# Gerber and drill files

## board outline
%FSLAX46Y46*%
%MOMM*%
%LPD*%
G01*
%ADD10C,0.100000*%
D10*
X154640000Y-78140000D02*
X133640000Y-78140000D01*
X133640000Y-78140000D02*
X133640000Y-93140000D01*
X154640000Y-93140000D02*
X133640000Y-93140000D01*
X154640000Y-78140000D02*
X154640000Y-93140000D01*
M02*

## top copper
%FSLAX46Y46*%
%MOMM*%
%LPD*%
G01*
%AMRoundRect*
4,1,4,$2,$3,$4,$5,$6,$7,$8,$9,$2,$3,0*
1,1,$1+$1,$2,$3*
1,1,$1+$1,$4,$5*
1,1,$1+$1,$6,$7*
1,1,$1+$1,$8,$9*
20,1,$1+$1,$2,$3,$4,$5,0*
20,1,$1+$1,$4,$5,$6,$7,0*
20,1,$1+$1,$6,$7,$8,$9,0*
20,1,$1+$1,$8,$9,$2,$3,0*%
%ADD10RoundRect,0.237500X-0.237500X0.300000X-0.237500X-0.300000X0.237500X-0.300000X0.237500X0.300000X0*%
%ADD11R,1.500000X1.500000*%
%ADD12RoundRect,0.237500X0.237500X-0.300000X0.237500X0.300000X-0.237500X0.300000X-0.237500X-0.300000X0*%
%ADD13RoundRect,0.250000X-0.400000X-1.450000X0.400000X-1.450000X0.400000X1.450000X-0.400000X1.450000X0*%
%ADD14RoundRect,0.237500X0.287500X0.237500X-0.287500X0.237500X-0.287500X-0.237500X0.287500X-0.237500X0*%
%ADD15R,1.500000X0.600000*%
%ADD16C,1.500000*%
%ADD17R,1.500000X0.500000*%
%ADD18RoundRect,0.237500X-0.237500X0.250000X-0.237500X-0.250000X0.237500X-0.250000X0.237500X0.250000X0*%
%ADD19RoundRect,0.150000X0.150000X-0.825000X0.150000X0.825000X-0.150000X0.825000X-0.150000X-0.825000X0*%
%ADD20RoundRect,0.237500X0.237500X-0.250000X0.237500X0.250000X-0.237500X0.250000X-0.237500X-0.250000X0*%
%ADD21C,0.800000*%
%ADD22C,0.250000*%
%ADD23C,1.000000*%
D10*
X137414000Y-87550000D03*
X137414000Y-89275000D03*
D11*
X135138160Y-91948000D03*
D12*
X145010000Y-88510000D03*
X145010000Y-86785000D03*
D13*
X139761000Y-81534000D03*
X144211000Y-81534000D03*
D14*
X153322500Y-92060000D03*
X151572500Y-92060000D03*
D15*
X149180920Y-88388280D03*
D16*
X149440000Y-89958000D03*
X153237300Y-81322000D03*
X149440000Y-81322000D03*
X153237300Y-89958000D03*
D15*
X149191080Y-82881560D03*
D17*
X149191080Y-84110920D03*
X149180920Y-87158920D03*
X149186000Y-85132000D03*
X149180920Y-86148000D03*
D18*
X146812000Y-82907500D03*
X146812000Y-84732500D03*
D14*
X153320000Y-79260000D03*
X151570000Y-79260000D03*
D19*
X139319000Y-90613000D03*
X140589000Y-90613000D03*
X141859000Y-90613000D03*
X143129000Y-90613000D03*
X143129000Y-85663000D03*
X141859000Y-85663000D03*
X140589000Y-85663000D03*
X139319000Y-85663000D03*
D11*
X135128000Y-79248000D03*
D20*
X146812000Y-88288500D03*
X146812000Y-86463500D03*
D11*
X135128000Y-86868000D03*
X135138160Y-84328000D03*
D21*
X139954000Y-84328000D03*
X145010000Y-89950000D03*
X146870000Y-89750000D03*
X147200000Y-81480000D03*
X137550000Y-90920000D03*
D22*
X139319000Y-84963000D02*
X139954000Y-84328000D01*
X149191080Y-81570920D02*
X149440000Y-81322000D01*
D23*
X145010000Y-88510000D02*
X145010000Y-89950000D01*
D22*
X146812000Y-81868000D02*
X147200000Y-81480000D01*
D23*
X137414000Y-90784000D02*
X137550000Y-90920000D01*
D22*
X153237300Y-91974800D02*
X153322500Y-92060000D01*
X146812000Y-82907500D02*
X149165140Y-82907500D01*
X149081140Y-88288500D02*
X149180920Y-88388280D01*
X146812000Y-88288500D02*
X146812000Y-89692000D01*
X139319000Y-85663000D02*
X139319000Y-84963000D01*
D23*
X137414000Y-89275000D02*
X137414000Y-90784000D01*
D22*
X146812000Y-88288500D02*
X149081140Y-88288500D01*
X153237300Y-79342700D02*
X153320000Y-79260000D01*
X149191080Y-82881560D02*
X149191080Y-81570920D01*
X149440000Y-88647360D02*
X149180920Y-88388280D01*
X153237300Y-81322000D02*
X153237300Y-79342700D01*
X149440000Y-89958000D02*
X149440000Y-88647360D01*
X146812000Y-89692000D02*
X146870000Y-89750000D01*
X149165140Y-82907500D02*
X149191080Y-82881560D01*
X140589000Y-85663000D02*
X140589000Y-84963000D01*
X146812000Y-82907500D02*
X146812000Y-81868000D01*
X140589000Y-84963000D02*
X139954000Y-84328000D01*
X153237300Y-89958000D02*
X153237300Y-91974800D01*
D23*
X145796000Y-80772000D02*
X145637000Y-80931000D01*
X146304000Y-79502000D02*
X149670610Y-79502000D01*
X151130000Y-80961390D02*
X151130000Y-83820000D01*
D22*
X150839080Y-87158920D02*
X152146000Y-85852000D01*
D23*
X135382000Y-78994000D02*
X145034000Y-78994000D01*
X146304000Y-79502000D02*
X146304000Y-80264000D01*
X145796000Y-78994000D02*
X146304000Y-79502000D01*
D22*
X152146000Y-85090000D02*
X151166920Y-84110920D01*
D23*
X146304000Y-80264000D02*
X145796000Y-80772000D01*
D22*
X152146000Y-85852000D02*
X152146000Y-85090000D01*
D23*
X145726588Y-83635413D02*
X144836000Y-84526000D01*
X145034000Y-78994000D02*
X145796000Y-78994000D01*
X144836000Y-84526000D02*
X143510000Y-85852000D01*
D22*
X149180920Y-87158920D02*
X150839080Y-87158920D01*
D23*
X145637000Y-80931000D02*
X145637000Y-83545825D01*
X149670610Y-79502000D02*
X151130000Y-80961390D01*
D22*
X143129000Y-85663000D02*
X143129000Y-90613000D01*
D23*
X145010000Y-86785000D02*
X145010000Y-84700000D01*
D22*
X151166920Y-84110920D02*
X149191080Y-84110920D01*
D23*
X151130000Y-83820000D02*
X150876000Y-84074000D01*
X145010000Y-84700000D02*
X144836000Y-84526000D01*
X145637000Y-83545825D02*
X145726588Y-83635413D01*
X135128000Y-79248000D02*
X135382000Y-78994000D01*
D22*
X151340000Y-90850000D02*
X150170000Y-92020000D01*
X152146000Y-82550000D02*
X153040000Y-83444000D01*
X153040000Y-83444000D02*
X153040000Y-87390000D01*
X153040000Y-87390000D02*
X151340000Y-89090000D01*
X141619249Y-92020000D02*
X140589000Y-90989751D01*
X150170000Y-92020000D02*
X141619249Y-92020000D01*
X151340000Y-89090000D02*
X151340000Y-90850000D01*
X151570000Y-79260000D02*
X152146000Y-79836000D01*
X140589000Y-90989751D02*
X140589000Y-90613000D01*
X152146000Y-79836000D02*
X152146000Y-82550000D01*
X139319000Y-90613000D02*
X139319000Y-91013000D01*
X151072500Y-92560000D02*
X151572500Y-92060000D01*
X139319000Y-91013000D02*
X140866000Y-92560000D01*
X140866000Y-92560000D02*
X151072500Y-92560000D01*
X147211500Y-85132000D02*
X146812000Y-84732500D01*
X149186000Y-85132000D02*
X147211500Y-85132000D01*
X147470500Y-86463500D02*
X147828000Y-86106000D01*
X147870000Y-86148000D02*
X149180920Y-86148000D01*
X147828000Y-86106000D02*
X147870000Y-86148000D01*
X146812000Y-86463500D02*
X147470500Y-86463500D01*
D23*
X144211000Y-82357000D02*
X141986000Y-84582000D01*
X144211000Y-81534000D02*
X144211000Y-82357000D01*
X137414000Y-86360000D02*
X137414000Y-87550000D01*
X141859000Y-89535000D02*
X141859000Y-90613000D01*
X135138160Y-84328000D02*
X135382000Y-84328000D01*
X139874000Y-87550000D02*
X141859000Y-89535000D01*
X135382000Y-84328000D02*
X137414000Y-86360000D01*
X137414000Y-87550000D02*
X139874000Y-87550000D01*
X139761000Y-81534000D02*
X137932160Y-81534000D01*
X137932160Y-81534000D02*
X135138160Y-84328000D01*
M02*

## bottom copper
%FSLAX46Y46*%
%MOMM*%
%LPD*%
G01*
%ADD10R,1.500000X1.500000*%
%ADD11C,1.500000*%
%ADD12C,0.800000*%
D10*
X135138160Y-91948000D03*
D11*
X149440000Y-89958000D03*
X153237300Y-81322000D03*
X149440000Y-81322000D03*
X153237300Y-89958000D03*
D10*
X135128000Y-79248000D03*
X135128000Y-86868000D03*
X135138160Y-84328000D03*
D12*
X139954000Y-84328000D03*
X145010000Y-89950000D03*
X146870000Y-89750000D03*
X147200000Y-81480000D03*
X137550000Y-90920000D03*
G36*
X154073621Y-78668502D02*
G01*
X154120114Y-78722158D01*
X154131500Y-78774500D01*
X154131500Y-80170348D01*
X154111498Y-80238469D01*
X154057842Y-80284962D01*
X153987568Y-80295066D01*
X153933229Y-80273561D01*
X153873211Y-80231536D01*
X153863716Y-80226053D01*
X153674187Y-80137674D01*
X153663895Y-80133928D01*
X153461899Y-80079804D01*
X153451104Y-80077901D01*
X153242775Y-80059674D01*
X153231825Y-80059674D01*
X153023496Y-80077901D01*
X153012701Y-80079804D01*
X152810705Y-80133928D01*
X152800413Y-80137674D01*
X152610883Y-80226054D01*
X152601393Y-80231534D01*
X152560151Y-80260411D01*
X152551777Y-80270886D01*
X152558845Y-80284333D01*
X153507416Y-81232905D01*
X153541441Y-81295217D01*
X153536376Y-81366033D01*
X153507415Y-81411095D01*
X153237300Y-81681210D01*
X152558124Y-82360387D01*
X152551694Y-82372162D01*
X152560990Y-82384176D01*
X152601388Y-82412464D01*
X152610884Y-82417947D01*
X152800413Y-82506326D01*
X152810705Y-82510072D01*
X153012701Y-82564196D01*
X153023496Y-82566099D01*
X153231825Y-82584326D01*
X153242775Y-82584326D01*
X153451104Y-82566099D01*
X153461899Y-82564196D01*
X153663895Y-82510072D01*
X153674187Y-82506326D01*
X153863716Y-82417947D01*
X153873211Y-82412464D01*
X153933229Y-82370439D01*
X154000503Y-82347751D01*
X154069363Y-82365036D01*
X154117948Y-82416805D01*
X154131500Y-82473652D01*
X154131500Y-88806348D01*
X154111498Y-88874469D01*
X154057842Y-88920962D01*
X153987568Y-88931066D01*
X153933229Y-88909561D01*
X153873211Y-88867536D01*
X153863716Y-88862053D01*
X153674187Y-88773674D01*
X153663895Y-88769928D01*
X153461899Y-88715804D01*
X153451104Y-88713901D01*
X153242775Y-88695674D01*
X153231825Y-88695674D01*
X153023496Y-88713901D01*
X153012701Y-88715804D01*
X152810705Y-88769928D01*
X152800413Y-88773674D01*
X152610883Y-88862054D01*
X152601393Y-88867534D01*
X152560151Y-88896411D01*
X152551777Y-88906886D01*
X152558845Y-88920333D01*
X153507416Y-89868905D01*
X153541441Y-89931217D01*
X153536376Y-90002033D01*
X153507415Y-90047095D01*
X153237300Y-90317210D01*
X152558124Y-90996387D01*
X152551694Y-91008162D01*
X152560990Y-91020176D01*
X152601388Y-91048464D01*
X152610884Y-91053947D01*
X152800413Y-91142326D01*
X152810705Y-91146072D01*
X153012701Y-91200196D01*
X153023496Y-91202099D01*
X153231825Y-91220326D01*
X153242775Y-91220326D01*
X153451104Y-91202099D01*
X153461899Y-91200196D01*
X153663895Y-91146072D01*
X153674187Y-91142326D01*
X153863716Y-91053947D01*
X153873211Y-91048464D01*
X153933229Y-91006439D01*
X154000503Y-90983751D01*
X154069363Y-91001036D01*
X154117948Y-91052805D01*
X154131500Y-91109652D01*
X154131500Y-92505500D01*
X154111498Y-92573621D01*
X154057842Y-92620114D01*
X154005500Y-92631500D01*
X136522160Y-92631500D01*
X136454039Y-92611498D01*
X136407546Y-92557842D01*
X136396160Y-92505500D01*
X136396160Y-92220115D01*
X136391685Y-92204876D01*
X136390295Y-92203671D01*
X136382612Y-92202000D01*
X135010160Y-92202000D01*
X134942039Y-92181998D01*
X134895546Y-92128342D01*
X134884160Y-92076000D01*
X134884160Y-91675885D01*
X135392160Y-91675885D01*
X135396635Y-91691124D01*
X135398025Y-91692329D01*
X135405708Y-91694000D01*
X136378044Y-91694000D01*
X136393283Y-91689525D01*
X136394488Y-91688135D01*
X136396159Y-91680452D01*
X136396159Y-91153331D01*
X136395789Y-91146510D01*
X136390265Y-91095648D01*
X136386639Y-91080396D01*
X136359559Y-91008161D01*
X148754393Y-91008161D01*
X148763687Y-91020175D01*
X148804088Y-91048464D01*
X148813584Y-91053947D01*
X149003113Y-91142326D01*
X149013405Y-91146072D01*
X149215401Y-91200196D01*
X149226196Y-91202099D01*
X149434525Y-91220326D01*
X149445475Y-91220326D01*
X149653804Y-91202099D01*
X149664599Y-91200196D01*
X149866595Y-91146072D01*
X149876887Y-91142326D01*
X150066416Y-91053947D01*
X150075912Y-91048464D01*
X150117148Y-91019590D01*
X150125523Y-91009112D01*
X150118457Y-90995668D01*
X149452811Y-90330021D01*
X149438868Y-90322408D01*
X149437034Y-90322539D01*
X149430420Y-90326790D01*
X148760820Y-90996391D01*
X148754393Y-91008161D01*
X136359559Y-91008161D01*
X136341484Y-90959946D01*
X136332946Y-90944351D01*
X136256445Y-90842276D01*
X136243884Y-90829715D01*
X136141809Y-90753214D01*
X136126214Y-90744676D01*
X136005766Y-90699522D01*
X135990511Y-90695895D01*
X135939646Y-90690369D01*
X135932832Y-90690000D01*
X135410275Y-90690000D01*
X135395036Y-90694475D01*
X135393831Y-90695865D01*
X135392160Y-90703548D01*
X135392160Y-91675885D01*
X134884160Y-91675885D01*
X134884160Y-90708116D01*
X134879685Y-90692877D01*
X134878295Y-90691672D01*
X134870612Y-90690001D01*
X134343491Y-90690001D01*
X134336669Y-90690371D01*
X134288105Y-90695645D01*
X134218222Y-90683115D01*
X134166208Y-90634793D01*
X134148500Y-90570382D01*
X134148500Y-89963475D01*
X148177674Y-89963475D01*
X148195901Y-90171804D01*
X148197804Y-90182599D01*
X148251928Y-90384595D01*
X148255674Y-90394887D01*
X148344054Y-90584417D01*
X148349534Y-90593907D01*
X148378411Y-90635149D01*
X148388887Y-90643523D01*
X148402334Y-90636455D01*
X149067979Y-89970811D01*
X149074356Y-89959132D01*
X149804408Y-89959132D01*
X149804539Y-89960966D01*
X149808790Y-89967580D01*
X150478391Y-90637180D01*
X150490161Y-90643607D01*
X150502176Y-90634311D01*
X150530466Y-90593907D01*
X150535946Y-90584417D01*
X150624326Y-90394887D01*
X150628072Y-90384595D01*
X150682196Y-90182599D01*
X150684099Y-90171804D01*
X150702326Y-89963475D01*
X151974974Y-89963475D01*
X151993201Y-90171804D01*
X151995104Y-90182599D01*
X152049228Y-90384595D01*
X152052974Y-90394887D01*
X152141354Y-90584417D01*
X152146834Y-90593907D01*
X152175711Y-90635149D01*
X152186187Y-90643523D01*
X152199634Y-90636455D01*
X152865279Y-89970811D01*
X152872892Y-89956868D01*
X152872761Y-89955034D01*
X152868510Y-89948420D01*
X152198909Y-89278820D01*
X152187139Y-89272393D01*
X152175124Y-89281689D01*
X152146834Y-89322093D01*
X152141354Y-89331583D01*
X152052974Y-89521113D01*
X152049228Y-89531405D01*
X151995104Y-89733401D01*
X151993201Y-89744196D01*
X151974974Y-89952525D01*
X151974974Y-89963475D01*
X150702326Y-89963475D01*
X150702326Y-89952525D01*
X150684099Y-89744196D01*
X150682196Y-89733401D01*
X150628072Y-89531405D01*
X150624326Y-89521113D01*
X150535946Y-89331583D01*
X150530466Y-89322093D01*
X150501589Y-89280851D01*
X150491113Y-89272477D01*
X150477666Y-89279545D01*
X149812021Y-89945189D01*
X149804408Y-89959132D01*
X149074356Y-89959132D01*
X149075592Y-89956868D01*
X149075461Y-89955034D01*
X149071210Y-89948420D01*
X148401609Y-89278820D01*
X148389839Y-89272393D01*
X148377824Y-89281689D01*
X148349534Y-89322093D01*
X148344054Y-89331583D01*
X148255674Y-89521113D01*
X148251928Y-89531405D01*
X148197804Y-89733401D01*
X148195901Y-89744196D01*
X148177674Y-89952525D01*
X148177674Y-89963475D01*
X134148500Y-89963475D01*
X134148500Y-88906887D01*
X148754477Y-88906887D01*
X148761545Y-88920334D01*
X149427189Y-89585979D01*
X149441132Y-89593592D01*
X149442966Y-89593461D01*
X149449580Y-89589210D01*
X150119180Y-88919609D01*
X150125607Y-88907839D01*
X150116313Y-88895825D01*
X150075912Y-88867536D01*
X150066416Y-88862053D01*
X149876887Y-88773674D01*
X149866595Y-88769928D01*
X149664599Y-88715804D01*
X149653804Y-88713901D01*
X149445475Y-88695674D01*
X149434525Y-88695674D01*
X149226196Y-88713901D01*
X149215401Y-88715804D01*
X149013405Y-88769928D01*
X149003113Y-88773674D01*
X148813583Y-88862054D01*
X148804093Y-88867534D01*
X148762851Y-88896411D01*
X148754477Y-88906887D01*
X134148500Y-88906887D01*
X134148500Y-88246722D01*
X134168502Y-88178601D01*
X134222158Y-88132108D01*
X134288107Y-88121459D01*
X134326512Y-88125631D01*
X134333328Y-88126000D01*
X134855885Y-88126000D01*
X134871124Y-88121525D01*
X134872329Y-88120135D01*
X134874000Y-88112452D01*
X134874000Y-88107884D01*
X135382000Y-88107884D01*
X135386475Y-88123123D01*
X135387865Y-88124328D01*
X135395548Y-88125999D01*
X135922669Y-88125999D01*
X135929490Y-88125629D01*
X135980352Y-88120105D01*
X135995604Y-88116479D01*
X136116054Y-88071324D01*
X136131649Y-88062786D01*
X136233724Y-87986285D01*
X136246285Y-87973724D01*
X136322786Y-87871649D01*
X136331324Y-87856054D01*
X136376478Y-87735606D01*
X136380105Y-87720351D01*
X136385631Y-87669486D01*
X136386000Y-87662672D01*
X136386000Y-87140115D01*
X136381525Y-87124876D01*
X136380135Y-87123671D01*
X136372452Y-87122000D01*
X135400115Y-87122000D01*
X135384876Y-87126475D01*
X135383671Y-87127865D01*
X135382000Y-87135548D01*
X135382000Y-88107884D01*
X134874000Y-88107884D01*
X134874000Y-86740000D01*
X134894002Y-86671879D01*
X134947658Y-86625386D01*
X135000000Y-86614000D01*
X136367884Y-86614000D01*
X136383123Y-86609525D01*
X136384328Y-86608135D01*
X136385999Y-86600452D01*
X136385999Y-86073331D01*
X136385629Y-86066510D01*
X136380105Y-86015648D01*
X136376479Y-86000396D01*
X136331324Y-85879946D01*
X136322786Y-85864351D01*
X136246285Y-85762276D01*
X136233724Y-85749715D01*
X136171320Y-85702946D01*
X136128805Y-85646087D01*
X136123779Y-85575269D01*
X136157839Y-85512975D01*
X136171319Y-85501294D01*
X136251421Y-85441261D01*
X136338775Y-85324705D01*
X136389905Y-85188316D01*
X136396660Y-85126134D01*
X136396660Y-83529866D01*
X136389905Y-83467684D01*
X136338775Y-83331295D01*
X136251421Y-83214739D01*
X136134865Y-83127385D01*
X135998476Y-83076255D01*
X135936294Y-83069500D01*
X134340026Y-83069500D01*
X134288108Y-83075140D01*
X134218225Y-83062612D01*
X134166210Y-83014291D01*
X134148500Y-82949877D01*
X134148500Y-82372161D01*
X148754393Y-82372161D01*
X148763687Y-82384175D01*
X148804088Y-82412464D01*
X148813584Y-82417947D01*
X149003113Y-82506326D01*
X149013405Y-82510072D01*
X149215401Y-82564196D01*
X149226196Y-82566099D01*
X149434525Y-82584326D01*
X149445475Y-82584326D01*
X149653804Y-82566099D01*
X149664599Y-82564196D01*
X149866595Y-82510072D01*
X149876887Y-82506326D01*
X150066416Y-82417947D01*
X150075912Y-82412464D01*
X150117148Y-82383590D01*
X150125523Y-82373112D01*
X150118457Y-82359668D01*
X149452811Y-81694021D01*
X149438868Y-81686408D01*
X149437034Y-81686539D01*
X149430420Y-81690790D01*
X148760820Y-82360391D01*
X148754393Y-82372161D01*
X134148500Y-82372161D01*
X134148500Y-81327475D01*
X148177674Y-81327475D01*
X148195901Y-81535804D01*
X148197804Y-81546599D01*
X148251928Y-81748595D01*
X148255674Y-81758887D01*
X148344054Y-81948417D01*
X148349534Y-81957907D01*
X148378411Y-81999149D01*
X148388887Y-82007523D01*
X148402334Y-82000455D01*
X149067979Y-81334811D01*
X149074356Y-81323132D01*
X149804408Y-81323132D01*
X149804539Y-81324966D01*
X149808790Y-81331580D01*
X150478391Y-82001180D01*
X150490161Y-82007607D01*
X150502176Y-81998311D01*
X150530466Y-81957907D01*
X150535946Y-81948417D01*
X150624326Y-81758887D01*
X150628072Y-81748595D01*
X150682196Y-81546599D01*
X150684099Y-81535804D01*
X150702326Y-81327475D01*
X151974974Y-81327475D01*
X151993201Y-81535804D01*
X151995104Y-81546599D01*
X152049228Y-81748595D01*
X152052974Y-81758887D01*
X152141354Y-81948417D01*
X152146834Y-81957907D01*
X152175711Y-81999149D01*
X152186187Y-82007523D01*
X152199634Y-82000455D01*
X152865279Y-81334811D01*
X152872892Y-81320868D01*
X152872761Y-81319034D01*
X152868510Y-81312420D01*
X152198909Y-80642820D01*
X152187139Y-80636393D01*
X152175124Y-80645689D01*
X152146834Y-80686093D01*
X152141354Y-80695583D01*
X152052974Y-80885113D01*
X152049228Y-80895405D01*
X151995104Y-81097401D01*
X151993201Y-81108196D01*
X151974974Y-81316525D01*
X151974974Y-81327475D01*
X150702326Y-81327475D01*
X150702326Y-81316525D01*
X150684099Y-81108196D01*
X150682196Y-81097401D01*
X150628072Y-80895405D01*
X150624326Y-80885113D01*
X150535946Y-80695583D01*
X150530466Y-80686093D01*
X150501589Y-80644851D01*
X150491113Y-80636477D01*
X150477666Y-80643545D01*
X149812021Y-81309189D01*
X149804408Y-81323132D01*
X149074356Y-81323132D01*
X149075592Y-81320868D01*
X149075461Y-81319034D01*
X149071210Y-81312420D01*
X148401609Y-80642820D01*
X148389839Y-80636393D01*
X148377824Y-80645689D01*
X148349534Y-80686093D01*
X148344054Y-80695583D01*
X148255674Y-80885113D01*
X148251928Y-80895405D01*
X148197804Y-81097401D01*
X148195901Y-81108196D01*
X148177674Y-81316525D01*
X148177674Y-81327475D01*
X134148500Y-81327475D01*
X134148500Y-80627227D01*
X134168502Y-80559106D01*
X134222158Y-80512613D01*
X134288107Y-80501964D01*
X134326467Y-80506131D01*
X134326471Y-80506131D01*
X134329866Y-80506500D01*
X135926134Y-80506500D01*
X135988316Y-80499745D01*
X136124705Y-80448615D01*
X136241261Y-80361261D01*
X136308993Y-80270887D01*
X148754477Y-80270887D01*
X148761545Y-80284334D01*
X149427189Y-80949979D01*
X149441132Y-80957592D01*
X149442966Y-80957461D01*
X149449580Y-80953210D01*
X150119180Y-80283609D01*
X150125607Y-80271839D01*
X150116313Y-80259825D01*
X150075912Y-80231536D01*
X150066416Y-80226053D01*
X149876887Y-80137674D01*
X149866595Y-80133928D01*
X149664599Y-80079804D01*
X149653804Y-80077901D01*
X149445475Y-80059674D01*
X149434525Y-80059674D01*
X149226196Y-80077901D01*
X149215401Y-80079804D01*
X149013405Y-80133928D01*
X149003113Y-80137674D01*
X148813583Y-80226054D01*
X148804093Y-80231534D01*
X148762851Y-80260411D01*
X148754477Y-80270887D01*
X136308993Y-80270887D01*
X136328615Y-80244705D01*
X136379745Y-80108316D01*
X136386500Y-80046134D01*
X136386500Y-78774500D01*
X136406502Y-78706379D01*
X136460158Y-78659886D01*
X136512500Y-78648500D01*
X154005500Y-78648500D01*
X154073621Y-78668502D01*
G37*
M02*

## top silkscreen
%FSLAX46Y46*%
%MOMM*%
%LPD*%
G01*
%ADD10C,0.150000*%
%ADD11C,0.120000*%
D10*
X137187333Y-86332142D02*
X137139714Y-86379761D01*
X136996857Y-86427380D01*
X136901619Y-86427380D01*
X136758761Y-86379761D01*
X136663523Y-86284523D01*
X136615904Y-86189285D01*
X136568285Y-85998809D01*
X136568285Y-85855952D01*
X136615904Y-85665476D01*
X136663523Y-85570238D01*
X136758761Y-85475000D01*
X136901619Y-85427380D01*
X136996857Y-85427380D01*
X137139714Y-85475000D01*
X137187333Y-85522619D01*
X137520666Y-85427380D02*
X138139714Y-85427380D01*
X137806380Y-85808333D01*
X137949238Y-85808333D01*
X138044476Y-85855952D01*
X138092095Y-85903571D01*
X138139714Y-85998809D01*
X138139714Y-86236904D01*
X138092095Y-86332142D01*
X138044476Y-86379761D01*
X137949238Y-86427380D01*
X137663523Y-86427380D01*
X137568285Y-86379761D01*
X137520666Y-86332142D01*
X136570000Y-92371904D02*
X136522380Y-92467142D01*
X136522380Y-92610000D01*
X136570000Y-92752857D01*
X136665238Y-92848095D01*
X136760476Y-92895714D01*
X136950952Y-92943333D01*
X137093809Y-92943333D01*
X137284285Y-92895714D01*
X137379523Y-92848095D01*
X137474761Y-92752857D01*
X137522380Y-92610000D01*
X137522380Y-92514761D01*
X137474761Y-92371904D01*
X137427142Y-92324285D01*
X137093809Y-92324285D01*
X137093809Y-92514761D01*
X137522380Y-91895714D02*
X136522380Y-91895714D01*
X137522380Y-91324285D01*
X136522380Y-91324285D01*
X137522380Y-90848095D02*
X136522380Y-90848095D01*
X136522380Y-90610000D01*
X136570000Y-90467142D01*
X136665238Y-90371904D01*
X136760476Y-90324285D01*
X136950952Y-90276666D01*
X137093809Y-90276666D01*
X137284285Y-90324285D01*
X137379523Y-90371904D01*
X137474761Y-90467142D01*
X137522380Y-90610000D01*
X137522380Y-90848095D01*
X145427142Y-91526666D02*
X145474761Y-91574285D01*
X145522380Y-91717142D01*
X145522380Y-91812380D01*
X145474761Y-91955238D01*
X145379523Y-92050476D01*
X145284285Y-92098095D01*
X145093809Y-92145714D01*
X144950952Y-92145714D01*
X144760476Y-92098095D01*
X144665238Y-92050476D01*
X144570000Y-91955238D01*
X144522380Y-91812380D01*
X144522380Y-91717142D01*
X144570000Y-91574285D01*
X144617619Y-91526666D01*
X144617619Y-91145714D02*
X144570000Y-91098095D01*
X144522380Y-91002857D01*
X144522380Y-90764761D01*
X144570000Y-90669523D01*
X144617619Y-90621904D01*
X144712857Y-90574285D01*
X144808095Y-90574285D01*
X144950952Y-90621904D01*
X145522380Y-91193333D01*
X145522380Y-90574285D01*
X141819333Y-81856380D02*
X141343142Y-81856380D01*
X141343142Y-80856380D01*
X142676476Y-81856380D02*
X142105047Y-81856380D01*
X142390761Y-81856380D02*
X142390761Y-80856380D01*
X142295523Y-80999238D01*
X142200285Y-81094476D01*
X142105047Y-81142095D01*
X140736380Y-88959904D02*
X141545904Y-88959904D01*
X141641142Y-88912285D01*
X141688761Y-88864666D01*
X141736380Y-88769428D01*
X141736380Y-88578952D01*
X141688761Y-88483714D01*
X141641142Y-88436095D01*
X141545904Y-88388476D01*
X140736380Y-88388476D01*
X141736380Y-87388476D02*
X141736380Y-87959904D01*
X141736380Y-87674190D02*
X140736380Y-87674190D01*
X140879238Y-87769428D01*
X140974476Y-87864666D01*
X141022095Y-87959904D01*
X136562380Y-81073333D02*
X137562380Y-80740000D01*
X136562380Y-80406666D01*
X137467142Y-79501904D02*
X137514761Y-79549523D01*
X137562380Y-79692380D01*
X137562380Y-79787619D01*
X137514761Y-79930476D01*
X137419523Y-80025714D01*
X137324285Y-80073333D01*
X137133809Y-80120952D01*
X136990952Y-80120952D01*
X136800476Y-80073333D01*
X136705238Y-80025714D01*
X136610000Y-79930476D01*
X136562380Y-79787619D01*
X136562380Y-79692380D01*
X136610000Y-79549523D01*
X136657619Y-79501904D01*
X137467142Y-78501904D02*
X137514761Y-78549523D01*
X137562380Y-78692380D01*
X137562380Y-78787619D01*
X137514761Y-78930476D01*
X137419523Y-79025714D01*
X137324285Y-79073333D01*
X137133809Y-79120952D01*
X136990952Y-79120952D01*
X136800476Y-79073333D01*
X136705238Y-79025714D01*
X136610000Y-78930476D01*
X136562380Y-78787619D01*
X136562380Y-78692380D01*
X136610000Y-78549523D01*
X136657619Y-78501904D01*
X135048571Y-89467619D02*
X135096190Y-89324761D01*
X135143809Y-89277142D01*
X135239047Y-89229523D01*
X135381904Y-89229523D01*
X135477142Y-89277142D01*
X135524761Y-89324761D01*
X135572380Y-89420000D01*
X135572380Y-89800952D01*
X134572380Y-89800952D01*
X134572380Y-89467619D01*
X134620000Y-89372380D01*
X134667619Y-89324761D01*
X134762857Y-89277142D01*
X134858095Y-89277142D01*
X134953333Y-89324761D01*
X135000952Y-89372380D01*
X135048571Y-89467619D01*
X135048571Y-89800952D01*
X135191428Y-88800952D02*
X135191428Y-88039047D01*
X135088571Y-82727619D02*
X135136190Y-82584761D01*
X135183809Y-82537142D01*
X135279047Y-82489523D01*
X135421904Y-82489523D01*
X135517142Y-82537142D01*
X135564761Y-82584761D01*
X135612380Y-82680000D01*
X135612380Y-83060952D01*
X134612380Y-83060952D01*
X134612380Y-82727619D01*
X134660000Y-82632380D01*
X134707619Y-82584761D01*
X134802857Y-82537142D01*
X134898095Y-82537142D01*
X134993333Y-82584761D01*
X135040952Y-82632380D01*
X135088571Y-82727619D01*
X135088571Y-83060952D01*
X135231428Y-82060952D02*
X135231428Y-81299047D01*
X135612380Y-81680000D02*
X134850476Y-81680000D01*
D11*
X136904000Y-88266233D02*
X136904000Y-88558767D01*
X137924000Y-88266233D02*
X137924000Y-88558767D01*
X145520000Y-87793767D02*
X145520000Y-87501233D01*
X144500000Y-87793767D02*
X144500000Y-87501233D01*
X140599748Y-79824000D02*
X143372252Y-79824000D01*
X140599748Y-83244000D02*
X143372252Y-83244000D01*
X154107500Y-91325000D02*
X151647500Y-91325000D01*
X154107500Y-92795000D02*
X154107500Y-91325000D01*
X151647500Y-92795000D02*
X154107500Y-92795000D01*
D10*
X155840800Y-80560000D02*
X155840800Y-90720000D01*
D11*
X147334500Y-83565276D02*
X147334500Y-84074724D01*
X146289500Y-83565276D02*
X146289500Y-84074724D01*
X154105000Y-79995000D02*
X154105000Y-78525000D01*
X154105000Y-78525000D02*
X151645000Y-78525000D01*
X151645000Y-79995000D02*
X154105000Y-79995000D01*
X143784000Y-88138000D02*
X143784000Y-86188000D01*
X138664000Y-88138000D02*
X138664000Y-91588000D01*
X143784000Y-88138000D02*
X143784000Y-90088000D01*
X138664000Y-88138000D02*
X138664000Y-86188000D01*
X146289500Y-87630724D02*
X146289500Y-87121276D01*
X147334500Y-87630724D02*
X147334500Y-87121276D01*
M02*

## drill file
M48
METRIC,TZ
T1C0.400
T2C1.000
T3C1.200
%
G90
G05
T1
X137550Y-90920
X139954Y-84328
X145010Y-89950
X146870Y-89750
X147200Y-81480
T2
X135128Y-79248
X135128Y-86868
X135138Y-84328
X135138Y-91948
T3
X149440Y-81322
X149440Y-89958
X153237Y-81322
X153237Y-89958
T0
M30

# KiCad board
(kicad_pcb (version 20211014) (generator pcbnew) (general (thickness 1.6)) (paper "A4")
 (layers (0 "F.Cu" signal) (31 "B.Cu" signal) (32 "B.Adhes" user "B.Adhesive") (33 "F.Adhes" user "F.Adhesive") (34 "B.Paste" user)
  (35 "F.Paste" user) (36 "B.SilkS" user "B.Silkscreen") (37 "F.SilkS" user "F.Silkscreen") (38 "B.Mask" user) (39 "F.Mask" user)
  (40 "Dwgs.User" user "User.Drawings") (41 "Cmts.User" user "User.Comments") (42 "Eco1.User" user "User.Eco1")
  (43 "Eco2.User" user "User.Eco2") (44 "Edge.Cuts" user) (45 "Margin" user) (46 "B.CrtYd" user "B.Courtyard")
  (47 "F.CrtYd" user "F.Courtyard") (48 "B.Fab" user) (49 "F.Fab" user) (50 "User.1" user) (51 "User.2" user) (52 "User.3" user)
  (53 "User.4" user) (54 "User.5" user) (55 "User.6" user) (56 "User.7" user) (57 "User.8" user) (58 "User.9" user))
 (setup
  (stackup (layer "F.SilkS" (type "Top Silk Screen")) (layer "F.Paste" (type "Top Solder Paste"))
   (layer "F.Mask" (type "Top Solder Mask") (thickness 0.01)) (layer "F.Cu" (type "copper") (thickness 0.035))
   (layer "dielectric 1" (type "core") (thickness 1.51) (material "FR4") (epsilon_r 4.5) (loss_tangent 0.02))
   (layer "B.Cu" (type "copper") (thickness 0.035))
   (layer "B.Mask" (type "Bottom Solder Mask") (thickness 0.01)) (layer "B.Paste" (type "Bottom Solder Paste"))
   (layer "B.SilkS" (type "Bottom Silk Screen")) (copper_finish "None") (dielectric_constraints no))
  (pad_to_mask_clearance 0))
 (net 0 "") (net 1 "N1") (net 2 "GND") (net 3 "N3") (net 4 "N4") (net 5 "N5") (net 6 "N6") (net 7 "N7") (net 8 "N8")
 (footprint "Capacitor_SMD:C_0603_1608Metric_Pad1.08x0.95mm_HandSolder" (layer "F.Cu") (at 137.414 88.4125 -90)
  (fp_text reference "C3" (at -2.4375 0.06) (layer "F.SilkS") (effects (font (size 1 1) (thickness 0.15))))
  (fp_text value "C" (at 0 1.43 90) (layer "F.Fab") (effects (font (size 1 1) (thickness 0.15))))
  (fp_line (start -0.146267 0.51) (end 0.146267 0.51) (layer "F.SilkS") (width 0.12))
  (fp_line (start -0.146267 -0.51) (end 0.146267 -0.51) (layer "F.SilkS") (width 0.12))
  (pad "1" smd roundrect (at -0.8625 0 270) (size 1.075 0.95) (layers "F.Cu" "F.Paste" "F.Mask") (roundrect_rratio 0.25) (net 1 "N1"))
  (pad "2" smd roundrect (at 0.8625 0 270) (size 1.075 0.95) (layers "F.Cu" "F.Paste" "F.Mask") (roundrect_rratio 0.25) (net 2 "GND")))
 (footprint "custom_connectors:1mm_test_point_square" (layer "F.Cu") (at 135.128 91.948 -90)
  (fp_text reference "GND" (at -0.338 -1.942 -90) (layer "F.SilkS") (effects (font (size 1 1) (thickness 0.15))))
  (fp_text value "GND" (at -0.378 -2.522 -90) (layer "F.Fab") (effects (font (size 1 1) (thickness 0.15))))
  (pad "1" thru_hole rect (at 0 -0.01016 270) (size 1.5 1.5) (drill 1) (layers *.Cu *.Mask) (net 2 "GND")))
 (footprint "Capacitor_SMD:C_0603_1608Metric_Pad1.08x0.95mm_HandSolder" (layer "F.Cu") (at 145.01 87.6475 90)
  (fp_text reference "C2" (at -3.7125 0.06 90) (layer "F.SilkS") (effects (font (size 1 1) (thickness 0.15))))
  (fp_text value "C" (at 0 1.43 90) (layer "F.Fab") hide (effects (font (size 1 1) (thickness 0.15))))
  (fp_line (start -0.146267 0.51) (end 0.146267 0.51) (layer "F.SilkS") (width 0.12))
  (fp_line (start -0.146267 -0.51) (end 0.146267 -0.51) (layer "F.SilkS") (width 0.12))
  (pad "1" smd roundrect (at -0.8625 0 90) (size 1.075 0.95) (layers "F.Cu" "F.Paste" "F.Mask") (roundrect_rratio 0.25) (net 2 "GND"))
  (pad "2" smd roundrect (at 0.8625 0 90) (size 1.075 0.95) (layers "F.Cu" "F.Paste" "F.Mask") (roundrect_rratio 0.25) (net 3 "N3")))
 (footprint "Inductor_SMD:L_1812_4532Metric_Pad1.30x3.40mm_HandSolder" (layer "F.Cu") (at 141.986 81.534)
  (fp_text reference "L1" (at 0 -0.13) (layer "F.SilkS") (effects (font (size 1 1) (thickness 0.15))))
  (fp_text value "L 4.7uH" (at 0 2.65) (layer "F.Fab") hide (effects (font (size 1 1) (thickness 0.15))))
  (fp_line (start -1.386252 -1.71) (end 1.386252 -1.71) (layer "F.SilkS") (width 0.12))
  (fp_line (start -1.386252 1.71) (end 1.386252 1.71) (layer "F.SilkS") (width 0.12))
  (pad "1" smd roundrect (at -2.225 0) (size 1.3 3.4) (layers "F.Cu" "F.Paste" "F.Mask") (roundrect_rratio 0.1923076923) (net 1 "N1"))
  (pad "2" smd roundrect (at 2.225 0) (size 1.3 3.4) (layers "F.Cu" "F.Paste" "F.Mask") (roundrect_rratio 0.1923076923) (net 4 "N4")))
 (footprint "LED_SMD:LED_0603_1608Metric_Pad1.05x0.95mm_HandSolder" (layer "F.Cu") (at 152.4475 92.06 180)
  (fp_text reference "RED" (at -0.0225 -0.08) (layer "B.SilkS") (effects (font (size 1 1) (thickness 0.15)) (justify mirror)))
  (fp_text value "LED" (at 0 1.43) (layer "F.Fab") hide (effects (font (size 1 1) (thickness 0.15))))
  (fp_line (start -1.66 0.735) (end 0.8 0.735) (layer "F.SilkS") (width 0.12))
  (fp_line (start -1.66 -0.735) (end -1.66 0.735) (layer "F.SilkS") (width 0.12))
  (fp_line (start 0.8 -0.735) (end -1.66 -0.735) (layer "F.SilkS") (width 0.12))
  (pad "1" smd roundrect (at -0.875 0 180) (size 1.05 0.95) (layers "F.Cu" "F.Paste" "F.Mask") (roundrect_rratio 0.25) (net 2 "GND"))
  (pad "2" smd roundrect (at 0.875 0 180) (size 1.05 0.95) (layers "F.Cu" "F.Paste" "F.Mask") (roundrect_rratio 0.25) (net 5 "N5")))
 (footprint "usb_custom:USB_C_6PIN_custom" (layer "F.Cu") (at 149.44 85.64 -90)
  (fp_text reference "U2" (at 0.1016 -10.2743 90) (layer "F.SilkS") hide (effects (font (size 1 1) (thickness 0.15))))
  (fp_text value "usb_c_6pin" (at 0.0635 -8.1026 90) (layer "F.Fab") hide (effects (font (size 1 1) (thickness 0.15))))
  (fp_line (start -5.08 -6.4008) (end 5.08 -6.4008) (layer "F.SilkS") (width 0.15))
  (pad "1" smd rect locked (at 2.74828 0.25908 270) (size 0.6 1.5) (layers "F.Cu" "F.Paste" "F.Mask") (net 2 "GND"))
  (pad "1" thru_hole circle locked (at 4.318 0 270) (size 1.5 1.5) (drill 1.2) (layers *.Cu *.Mask) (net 2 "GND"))
  (pad "1" thru_hole circle locked (at -4.318 -3.7973 270) (size 1.5 1.5) (drill 1.2) (layers *.Cu *.Mask) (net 2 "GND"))
  (pad "1" thru_hole circle locked (at -4.318 0 270) (size 1.5 1.5) (drill 1.2) (layers *.Cu *.Mask) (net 2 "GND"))
  (pad "1" thru_hole circle locked (at 4.318 -3.7973 270) (size 1.5 1.5) (drill 1.2) (layers *.Cu *.Mask) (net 2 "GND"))
  (pad "1" smd rect locked (at -2.75844 0.24892 270) (size 0.6 1.5) (layers "F.Cu" "F.Paste" "F.Mask") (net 2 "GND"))
  (pad "2" smd rect locked (at -1.52908 0.24892 270) (size 0.5 1.5) (layers "F.Cu" "F.Paste" "F.Mask") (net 3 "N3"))
  (pad "2" smd rect locked (at 1.51892 0.25908 270) (size 0.5 1.5) (layers "F.Cu" "F.Paste" "F.Mask") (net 3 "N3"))
  (pad "3" smd rect locked (at -0.508 0.254 270) (size 0.5 1.5) (layers "F.Cu" "F.Paste" "F.Mask") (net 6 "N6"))
  (pad "4" smd rect locked (at 0.508 0.25908 270) (size 0.5 1.5) (layers "F.Cu" "F.Paste" "F.Mask") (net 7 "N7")))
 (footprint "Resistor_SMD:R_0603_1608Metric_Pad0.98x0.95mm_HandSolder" (layer "F.Cu") (at 146.812 83.82 -90)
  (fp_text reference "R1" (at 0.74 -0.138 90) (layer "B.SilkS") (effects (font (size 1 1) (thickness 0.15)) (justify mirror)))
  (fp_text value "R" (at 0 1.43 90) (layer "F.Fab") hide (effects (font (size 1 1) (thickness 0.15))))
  (fp_line (start -0.254724 -0.5225) (end 0.254724 -0.5225) (layer "F.SilkS") (width 0.12))
  (fp_line (start -0.254724 0.5225) (end 0.254724 0.5225) (layer "F.SilkS") (width 0.12))
  (pad "1" smd roundrect (at -0.9125 0 270) (size 0.975 0.95) (layers "F.Cu" "F.Paste" "F.Mask") (roundrect_rratio 0.25) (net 2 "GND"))
  (pad "2" smd roundrect (at 0.9125 0 270) (size 0.975 0.95) (layers "F.Cu" "F.Paste" "F.Mask") (roundrect_rratio 0.25) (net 6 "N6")))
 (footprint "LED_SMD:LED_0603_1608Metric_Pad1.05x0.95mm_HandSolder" (layer "F.Cu") (at 152.445 79.26 180)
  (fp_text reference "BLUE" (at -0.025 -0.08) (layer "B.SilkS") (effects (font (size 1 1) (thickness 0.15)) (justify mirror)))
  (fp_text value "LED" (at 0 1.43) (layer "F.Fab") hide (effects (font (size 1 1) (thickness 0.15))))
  (fp_line (start -1.66 -0.735) (end -1.66 0.735) (layer "F.SilkS") (width 0.12))
  (fp_line (start -1.66 0.735) (end 0.8 0.735) (layer "F.SilkS") (width 0.12))
  (fp_line (start 0.8 -0.735) (end -1.66 -0.735) (layer "F.SilkS") (width 0.12))
  (pad "1" smd roundrect (at -0.875 0 180) (size 1.05 0.95) (layers "F.Cu" "F.Paste" "F.Mask") (roundrect_rratio 0.25) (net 2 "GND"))
  (pad "2" smd roundrect (at 0.875 0 180) (size 1.05 0.95) (layers "F.Cu" "F.Paste" "F.Mask") (roundrect_rratio 0.25) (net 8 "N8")))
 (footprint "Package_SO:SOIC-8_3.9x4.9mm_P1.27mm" (layer "F.Cu") (at 141.224 88.138 90)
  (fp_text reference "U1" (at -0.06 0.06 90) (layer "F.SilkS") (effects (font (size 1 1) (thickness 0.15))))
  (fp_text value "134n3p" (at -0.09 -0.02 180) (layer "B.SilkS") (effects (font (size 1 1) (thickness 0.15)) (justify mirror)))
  (fp_line (start 0 2.56) (end 1.95 2.56) (layer "F.SilkS") (width 0.12))
  (fp_line (start 0 -2.56) (end -3.45 -2.56) (layer "F.SilkS") (width 0.12))
  (fp_line (start 0 2.56) (end -1.95 2.56) (layer "F.SilkS") (width 0.12))
  (fp_line (start 0 -2.56) (end 1.95 -2.56) (layer "F.SilkS") (width 0.12))
  (pad "1" smd roundrect (at -2.475 -1.905 90) (size 1.95 0.6) (layers "F.Cu" "F.Paste" "F.Mask") (roundrect_rratio 0.25) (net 5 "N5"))
  (pad "2" smd roundrect (at -2.475 -0.635 90) (size 1.95 0.6) (layers "F.Cu" "F.Paste" "F.Mask") (roundrect_rratio 0.25) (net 8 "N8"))
  (pad "3" smd roundrect (at -2.475 0.635 90) (size 1.95 0.6) (layers "F.Cu" "F.Paste" "F.Mask") (roundrect_rratio 0.25) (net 1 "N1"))
  (pad "4" smd roundrect (at -2.475 1.905 90) (size 1.95 0.6) (layers "F.Cu" "F.Paste" "F.Mask") (roundrect_rratio 0.25) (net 3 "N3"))
  (pad "5" smd roundrect (at 2.475 1.905 90) (size 1.95 0.6) (layers "F.Cu" "F.Paste" "F.Mask") (roundrect_rratio 0.25) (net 3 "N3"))
  (pad "6" smd roundrect (at 2.475 0.635 90) (size 1.95 0.6) (layers "F.Cu" "F.Paste" "F.Mask") (roundrect_rratio 0.25) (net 4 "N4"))
  (pad "7" smd roundrect (at 2.475 -0.635 90) (size 1.95 0.6) (layers "F.Cu" "F.Paste" "F.Mask") (roundrect_rratio 0.25) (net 2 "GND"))
  (pad "8" smd roundrect (at 2.475 -1.905 90) (size 1.95 0.6) (layers "F.Cu" "F.Paste" "F.Mask") (roundrect_rratio 0.25) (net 2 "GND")))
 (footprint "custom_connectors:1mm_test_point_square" (layer "F.Cu") (at 135.11784 79.248 -90)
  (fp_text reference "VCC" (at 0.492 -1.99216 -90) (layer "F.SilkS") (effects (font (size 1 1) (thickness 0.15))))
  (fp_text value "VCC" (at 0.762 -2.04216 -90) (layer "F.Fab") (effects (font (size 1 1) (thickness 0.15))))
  (pad "1" thru_hole rect (at 0 -0.01016 270) (size 1.5 1.5) (drill 1) (layers *.Cu *.Mask) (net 3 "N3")))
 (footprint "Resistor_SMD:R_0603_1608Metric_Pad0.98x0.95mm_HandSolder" (layer "F.Cu") (at 146.812 87.376 90)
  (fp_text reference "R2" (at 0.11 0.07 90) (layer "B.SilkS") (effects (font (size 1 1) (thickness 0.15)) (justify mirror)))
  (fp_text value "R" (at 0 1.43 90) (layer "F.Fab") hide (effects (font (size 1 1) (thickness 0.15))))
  (fp_line (start -0.254724 -0.5225) (end 0.254724 -0.5225) (layer "F.SilkS") (width 0.12))
  (fp_line (start -0.254724 0.5225) (end 0.254724 0.5225) (layer "F.SilkS") (width 0.12))
  (pad "1" smd roundrect (at -0.9125 0 90) (size 0.975 0.95) (layers "F.Cu" "F.Paste" "F.Mask") (roundrect_rratio 0.25) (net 2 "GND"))
  (pad "2" smd roundrect (at 0.9125 0 90) (size 0.975 0.95) (layers "F.Cu" "F.Paste" "F.Mask") (roundrect_rratio 0.25) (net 7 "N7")))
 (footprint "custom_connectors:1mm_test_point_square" (layer "F.Cu") (at 135.11784 86.868 -90)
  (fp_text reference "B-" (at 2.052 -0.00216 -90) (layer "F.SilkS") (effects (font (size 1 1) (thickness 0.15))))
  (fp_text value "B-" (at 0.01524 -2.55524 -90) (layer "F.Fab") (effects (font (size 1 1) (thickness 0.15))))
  (pad "1" thru_hole rect (at 0 -0.01016 270) (size 1.5 1.5) (drill 1) (layers *.Cu *.Mask) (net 2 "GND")))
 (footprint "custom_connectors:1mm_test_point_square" (layer "F.Cu") (at 135.128 84.328 -90)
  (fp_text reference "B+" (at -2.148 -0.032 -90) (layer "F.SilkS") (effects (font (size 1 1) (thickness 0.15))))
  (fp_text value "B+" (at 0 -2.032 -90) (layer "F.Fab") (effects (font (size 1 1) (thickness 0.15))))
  (pad "1" thru_hole rect (at 0 -0.01016 270) (size 1.5 1.5) (drill 1) (layers *.Cu *.Mask) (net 1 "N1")))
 (gr_line (start 154.64 78.14) (end 133.64 78.14) (layer "Edge.Cuts") (width 0.1))
 (gr_line (start 133.64 78.14) (end 133.64 93.14) (layer "Edge.Cuts") (width 0.1))
 (gr_line (start 154.64 93.14) (end 133.64 93.14) (layer "Edge.Cuts") (width 0.1))
 (gr_line (start 154.64 78.14) (end 154.64 93.14) (layer "Edge.Cuts") (width 0.1))
 (segment (start 139.319 84.963) (end 139.954 84.328) (width 0.25) (layer "F.Cu") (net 2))
 (segment (start 149.19108 81.57092) (end 149.44 81.322) (width 0.25) (layer "F.Cu") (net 2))
 (segment (start 145.01 88.51) (end 145.01 89.95) (width 1) (layer "F.Cu") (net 2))
 (segment (start 146.812 81.868) (end 147.2 81.48) (width 0.25) (layer "F.Cu") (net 2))
 (segment (start 137.414 90.784) (end 137.55 90.92) (width 1) (layer "F.Cu") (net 2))
 (segment (start 153.2373 91.9748) (end 153.3225 92.06) (width 0.25) (layer "F.Cu") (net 2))
 (segment (start 146.812 82.9075) (end 149.16514 82.9075) (width 0.25) (layer "F.Cu") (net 2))
 (segment (start 149.08114 88.2885) (end 149.18092 88.38828) (width 0.25) (layer "F.Cu") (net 2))
 (segment (start 146.812 88.2885) (end 146.812 89.692) (width 0.25) (layer "F.Cu") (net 2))
 (segment (start 139.319 85.663) (end 139.319 84.963) (width 0.25) (layer "F.Cu") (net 2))
 (segment (start 137.414 89.275) (end 137.414 90.784) (width 1) (layer "F.Cu") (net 2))
 (segment (start 146.812 88.2885) (end 149.08114 88.2885) (width 0.25) (layer "F.Cu") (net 2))
 (segment (start 153.2373 79.3427) (end 153.32 79.26) (width 0.25) (layer "F.Cu") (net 2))
 (segment (start 149.19108 82.88156) (end 149.19108 81.57092) (width 0.25) (layer "F.Cu") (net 2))
 (segment (start 149.44 88.64736) (end 149.18092 88.38828) (width 0.25) (layer "F.Cu") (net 2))
 (segment (start 153.2373 81.322) (end 153.2373 79.3427) (width 0.25) (layer "F.Cu") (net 2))
 (segment (start 149.44 89.958) (end 149.44 88.64736) (width 0.25) (layer "F.Cu") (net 2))
 (segment (start 146.812 89.692) (end 146.87 89.75) (width 0.25) (layer "F.Cu") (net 2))
 (segment (start 149.16514 82.9075) (end 149.19108 82.88156) (width 0.25) (layer "F.Cu") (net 2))
 (segment (start 140.589 85.663) (end 140.589 84.963) (width 0.25) (layer "F.Cu") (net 2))
 (segment (start 146.812 82.9075) (end 146.812 81.868) (width 0.25) (layer "F.Cu") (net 2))
 (segment (start 140.589 84.963) (end 139.954 84.328) (width 0.25) (layer "F.Cu") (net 2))
 (segment (start 153.2373 89.958) (end 153.2373 91.9748) (width 0.25) (layer "F.Cu") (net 2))
 (via (at 139.954 84.328) (size 0.8) (drill 0.4) (layers "F.Cu" "B.Cu") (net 2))
 (via (at 145.01 89.95) (size 0.8) (drill 0.4) (layers "F.Cu" "B.Cu") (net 2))
 (via (at 146.87 89.75) (size 0.8) (drill 0.4) (layers "F.Cu" "B.Cu") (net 2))
 (via (at 147.2 81.48) (size 0.8) (drill 0.4) (layers "F.Cu" "B.Cu") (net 2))
 (via (at 137.55 90.92) (size 0.8) (drill 0.4) (layers "F.Cu" "B.Cu") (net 2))
 (segment (start 145.796 80.772) (end 145.637 80.931) (width 1) (layer "F.Cu") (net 3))
 (segment (start 146.304 79.502) (end 149.67061 79.502) (width 1) (layer "F.Cu") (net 3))
 (segment (start 151.13 80.96139) (end 151.13 83.82) (width 1) (layer "F.Cu") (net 3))
 (segment (start 150.83908 87.15892) (end 152.146 85.852) (width 0.25) (layer "F.Cu") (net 3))
 (segment (start 135.382 78.994) (end 145.034 78.994) (width 1) (layer "F.Cu") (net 3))
 (segment (start 146.304 79.502) (end 146.304 80.264) (width 1) (layer "F.Cu") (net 3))
 (segment (start 145.796 78.994) (end 146.304 79.502) (width 1) (layer "F.Cu") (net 3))
 (segment (start 152.146 85.09) (end 151.16692 84.11092) (width 0.25) (layer "F.Cu") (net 3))
 (segment (start 146.304 80.264) (end 145.796 80.772) (width 1) (layer "F.Cu") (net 3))
 (segment (start 152.146 85.852) (end 152.146 85.09) (width 0.25) (layer "F.Cu") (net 3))
 (segment (start 145.726588 83.635413) (end 144.836 84.526) (width 1) (layer "F.Cu") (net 3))
 (segment (start 145.034 78.994) (end 145.796 78.994) (width 1) (layer "F.Cu") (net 3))
 (segment (start 144.836 84.526) (end 143.51 85.852) (width 1) (layer "F.Cu") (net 3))
 (segment (start 149.18092 87.15892) (end 150.83908 87.15892) (width 0.25) (layer "F.Cu") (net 3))
 (segment (start 145.637 80.931) (end 145.637 83.545825) (width 1) (layer "F.Cu") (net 3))
 (segment (start 149.67061 79.502) (end 151.13 80.96139) (width 1) (layer "F.Cu") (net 3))
 (segment (start 143.129 85.663) (end 143.129 90.613) (width 0.25) (layer "F.Cu") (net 3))
 (segment (start 145.01 86.785) (end 145.01 84.7) (width 1) (layer "F.Cu") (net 3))
 (segment (start 151.16692 84.11092) (end 149.19108 84.11092) (width 0.25) (layer "F.Cu") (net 3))
 (segment (start 151.13 83.82) (end 150.876 84.074) (width 1) (layer "F.Cu") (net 3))
 (segment (start 145.01 84.7) (end 144.836 84.526) (width 1) (layer "F.Cu") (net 3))
 (segment (start 145.637 83.545825) (end 145.726588 83.635413) (width 1) (layer "F.Cu") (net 3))
 (segment (start 135.128 79.248) (end 135.382 78.994) (width 1) (layer "F.Cu") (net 3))
 (segment (start 151.34 90.85) (end 150.17 92.02) (width 0.25) (layer "F.Cu") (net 8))
 (segment (start 152.146 82.55) (end 153.04 83.444) (width 0.25) (layer "F.Cu") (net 8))
 (segment (start 153.04 83.444) (end 153.04 87.39) (width 0.25) (layer "F.Cu") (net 8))
 (segment (start 153.04 87.39) (end 151.34 89.09) (width 0.25) (layer "F.Cu") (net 8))
 (segment (start 141.619249 92.02) (end 140.589 90.989751) (width 0.25) (layer "F.Cu") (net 8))
 (segment (start 150.17 92.02) (end 141.619249 92.02) (width 0.25) (layer "F.Cu") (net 8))
 (segment (start 151.34 89.09) (end 151.34 90.85) (width 0.25) (layer "F.Cu") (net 8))
 (segment (start 151.57 79.26) (end 152.146 79.836) (width 0.25) (layer "F.Cu") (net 8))
 (segment (start 140.589 90.989751) (end 140.589 90.613) (width 0.25) (layer "F.Cu") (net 8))
 (segment (start 152.146 79.836) (end 152.146 82.55) (width 0.25) (layer "F.Cu") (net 8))
 (segment (start 139.319 90.613) (end 139.319 91.013) (width 0.25) (layer "F.Cu") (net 5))
 (segment (start 151.0725 92.56) (end 151.5725 92.06) (width 0.25) (layer "F.Cu") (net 5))
 (segment (start 139.319 91.013) (end 140.866 92.56) (width 0.25) (layer "F.Cu") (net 5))
 (segment (start 140.866 92.56) (end 151.0725 92.56) (width 0.25) (layer "F.Cu") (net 5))
 (segment (start 147.2115 85.132) (end 146.812 84.7325) (width 0.25) (layer "F.Cu") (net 6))
 (segment (start 149.186 85.132) (end 147.2115 85.132) (width 0.25) (layer "F.Cu") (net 6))
 (segment (start 147.4705 86.4635) (end 147.828 86.106) (width 0.25) (layer "F.Cu") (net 7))
 (segment (start 147.87 86.148) (end 149.18092 86.148) (width 0.25) (layer "F.Cu") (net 7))
 (segment (start 147.828 86.106) (end 147.87 86.148) (width 0.25) (layer "F.Cu") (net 7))
 (segment (start 146.812 86.4635) (end 147.4705 86.4635) (width 0.25) (layer "F.Cu") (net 7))
 (segment (start 144.211 82.357) (end 141.986 84.582) (width 1) (layer "F.Cu") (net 4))
 (segment (start 144.211 81.534) (end 144.211 82.357) (width 1) (layer "F.Cu") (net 4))
 (segment (start 137.414 86.36) (end 137.414 87.55) (width 1) (layer "F.Cu") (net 1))
 (segment (start 141.859 89.535) (end 141.859 90.613) (width 1) (layer "F.Cu") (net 1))
 (segment (start 135.13816 84.328) (end 135.382 84.328) (width 1) (layer "F.Cu") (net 1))
 (segment (start 139.874 87.55) (end 141.859 89.535) (width 1) (layer "F.Cu") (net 1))
 (segment (start 135.382 84.328) (end 137.414 86.36) (width 1) (layer "F.Cu") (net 1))
 (segment (start 137.414 87.55) (end 139.874 87.55) (width 1) (layer "F.Cu") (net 1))
 (segment (start 139.761 81.534) (end 137.93216 81.534) (width 1) (layer "F.Cu") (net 1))
 (segment (start 137.93216 81.534) (end 135.13816 84.328) (width 1) (layer "F.Cu") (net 1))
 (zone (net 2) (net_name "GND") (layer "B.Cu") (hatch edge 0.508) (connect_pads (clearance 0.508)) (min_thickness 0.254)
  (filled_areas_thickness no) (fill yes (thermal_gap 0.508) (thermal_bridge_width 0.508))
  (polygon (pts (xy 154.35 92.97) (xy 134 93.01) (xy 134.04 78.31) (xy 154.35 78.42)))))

